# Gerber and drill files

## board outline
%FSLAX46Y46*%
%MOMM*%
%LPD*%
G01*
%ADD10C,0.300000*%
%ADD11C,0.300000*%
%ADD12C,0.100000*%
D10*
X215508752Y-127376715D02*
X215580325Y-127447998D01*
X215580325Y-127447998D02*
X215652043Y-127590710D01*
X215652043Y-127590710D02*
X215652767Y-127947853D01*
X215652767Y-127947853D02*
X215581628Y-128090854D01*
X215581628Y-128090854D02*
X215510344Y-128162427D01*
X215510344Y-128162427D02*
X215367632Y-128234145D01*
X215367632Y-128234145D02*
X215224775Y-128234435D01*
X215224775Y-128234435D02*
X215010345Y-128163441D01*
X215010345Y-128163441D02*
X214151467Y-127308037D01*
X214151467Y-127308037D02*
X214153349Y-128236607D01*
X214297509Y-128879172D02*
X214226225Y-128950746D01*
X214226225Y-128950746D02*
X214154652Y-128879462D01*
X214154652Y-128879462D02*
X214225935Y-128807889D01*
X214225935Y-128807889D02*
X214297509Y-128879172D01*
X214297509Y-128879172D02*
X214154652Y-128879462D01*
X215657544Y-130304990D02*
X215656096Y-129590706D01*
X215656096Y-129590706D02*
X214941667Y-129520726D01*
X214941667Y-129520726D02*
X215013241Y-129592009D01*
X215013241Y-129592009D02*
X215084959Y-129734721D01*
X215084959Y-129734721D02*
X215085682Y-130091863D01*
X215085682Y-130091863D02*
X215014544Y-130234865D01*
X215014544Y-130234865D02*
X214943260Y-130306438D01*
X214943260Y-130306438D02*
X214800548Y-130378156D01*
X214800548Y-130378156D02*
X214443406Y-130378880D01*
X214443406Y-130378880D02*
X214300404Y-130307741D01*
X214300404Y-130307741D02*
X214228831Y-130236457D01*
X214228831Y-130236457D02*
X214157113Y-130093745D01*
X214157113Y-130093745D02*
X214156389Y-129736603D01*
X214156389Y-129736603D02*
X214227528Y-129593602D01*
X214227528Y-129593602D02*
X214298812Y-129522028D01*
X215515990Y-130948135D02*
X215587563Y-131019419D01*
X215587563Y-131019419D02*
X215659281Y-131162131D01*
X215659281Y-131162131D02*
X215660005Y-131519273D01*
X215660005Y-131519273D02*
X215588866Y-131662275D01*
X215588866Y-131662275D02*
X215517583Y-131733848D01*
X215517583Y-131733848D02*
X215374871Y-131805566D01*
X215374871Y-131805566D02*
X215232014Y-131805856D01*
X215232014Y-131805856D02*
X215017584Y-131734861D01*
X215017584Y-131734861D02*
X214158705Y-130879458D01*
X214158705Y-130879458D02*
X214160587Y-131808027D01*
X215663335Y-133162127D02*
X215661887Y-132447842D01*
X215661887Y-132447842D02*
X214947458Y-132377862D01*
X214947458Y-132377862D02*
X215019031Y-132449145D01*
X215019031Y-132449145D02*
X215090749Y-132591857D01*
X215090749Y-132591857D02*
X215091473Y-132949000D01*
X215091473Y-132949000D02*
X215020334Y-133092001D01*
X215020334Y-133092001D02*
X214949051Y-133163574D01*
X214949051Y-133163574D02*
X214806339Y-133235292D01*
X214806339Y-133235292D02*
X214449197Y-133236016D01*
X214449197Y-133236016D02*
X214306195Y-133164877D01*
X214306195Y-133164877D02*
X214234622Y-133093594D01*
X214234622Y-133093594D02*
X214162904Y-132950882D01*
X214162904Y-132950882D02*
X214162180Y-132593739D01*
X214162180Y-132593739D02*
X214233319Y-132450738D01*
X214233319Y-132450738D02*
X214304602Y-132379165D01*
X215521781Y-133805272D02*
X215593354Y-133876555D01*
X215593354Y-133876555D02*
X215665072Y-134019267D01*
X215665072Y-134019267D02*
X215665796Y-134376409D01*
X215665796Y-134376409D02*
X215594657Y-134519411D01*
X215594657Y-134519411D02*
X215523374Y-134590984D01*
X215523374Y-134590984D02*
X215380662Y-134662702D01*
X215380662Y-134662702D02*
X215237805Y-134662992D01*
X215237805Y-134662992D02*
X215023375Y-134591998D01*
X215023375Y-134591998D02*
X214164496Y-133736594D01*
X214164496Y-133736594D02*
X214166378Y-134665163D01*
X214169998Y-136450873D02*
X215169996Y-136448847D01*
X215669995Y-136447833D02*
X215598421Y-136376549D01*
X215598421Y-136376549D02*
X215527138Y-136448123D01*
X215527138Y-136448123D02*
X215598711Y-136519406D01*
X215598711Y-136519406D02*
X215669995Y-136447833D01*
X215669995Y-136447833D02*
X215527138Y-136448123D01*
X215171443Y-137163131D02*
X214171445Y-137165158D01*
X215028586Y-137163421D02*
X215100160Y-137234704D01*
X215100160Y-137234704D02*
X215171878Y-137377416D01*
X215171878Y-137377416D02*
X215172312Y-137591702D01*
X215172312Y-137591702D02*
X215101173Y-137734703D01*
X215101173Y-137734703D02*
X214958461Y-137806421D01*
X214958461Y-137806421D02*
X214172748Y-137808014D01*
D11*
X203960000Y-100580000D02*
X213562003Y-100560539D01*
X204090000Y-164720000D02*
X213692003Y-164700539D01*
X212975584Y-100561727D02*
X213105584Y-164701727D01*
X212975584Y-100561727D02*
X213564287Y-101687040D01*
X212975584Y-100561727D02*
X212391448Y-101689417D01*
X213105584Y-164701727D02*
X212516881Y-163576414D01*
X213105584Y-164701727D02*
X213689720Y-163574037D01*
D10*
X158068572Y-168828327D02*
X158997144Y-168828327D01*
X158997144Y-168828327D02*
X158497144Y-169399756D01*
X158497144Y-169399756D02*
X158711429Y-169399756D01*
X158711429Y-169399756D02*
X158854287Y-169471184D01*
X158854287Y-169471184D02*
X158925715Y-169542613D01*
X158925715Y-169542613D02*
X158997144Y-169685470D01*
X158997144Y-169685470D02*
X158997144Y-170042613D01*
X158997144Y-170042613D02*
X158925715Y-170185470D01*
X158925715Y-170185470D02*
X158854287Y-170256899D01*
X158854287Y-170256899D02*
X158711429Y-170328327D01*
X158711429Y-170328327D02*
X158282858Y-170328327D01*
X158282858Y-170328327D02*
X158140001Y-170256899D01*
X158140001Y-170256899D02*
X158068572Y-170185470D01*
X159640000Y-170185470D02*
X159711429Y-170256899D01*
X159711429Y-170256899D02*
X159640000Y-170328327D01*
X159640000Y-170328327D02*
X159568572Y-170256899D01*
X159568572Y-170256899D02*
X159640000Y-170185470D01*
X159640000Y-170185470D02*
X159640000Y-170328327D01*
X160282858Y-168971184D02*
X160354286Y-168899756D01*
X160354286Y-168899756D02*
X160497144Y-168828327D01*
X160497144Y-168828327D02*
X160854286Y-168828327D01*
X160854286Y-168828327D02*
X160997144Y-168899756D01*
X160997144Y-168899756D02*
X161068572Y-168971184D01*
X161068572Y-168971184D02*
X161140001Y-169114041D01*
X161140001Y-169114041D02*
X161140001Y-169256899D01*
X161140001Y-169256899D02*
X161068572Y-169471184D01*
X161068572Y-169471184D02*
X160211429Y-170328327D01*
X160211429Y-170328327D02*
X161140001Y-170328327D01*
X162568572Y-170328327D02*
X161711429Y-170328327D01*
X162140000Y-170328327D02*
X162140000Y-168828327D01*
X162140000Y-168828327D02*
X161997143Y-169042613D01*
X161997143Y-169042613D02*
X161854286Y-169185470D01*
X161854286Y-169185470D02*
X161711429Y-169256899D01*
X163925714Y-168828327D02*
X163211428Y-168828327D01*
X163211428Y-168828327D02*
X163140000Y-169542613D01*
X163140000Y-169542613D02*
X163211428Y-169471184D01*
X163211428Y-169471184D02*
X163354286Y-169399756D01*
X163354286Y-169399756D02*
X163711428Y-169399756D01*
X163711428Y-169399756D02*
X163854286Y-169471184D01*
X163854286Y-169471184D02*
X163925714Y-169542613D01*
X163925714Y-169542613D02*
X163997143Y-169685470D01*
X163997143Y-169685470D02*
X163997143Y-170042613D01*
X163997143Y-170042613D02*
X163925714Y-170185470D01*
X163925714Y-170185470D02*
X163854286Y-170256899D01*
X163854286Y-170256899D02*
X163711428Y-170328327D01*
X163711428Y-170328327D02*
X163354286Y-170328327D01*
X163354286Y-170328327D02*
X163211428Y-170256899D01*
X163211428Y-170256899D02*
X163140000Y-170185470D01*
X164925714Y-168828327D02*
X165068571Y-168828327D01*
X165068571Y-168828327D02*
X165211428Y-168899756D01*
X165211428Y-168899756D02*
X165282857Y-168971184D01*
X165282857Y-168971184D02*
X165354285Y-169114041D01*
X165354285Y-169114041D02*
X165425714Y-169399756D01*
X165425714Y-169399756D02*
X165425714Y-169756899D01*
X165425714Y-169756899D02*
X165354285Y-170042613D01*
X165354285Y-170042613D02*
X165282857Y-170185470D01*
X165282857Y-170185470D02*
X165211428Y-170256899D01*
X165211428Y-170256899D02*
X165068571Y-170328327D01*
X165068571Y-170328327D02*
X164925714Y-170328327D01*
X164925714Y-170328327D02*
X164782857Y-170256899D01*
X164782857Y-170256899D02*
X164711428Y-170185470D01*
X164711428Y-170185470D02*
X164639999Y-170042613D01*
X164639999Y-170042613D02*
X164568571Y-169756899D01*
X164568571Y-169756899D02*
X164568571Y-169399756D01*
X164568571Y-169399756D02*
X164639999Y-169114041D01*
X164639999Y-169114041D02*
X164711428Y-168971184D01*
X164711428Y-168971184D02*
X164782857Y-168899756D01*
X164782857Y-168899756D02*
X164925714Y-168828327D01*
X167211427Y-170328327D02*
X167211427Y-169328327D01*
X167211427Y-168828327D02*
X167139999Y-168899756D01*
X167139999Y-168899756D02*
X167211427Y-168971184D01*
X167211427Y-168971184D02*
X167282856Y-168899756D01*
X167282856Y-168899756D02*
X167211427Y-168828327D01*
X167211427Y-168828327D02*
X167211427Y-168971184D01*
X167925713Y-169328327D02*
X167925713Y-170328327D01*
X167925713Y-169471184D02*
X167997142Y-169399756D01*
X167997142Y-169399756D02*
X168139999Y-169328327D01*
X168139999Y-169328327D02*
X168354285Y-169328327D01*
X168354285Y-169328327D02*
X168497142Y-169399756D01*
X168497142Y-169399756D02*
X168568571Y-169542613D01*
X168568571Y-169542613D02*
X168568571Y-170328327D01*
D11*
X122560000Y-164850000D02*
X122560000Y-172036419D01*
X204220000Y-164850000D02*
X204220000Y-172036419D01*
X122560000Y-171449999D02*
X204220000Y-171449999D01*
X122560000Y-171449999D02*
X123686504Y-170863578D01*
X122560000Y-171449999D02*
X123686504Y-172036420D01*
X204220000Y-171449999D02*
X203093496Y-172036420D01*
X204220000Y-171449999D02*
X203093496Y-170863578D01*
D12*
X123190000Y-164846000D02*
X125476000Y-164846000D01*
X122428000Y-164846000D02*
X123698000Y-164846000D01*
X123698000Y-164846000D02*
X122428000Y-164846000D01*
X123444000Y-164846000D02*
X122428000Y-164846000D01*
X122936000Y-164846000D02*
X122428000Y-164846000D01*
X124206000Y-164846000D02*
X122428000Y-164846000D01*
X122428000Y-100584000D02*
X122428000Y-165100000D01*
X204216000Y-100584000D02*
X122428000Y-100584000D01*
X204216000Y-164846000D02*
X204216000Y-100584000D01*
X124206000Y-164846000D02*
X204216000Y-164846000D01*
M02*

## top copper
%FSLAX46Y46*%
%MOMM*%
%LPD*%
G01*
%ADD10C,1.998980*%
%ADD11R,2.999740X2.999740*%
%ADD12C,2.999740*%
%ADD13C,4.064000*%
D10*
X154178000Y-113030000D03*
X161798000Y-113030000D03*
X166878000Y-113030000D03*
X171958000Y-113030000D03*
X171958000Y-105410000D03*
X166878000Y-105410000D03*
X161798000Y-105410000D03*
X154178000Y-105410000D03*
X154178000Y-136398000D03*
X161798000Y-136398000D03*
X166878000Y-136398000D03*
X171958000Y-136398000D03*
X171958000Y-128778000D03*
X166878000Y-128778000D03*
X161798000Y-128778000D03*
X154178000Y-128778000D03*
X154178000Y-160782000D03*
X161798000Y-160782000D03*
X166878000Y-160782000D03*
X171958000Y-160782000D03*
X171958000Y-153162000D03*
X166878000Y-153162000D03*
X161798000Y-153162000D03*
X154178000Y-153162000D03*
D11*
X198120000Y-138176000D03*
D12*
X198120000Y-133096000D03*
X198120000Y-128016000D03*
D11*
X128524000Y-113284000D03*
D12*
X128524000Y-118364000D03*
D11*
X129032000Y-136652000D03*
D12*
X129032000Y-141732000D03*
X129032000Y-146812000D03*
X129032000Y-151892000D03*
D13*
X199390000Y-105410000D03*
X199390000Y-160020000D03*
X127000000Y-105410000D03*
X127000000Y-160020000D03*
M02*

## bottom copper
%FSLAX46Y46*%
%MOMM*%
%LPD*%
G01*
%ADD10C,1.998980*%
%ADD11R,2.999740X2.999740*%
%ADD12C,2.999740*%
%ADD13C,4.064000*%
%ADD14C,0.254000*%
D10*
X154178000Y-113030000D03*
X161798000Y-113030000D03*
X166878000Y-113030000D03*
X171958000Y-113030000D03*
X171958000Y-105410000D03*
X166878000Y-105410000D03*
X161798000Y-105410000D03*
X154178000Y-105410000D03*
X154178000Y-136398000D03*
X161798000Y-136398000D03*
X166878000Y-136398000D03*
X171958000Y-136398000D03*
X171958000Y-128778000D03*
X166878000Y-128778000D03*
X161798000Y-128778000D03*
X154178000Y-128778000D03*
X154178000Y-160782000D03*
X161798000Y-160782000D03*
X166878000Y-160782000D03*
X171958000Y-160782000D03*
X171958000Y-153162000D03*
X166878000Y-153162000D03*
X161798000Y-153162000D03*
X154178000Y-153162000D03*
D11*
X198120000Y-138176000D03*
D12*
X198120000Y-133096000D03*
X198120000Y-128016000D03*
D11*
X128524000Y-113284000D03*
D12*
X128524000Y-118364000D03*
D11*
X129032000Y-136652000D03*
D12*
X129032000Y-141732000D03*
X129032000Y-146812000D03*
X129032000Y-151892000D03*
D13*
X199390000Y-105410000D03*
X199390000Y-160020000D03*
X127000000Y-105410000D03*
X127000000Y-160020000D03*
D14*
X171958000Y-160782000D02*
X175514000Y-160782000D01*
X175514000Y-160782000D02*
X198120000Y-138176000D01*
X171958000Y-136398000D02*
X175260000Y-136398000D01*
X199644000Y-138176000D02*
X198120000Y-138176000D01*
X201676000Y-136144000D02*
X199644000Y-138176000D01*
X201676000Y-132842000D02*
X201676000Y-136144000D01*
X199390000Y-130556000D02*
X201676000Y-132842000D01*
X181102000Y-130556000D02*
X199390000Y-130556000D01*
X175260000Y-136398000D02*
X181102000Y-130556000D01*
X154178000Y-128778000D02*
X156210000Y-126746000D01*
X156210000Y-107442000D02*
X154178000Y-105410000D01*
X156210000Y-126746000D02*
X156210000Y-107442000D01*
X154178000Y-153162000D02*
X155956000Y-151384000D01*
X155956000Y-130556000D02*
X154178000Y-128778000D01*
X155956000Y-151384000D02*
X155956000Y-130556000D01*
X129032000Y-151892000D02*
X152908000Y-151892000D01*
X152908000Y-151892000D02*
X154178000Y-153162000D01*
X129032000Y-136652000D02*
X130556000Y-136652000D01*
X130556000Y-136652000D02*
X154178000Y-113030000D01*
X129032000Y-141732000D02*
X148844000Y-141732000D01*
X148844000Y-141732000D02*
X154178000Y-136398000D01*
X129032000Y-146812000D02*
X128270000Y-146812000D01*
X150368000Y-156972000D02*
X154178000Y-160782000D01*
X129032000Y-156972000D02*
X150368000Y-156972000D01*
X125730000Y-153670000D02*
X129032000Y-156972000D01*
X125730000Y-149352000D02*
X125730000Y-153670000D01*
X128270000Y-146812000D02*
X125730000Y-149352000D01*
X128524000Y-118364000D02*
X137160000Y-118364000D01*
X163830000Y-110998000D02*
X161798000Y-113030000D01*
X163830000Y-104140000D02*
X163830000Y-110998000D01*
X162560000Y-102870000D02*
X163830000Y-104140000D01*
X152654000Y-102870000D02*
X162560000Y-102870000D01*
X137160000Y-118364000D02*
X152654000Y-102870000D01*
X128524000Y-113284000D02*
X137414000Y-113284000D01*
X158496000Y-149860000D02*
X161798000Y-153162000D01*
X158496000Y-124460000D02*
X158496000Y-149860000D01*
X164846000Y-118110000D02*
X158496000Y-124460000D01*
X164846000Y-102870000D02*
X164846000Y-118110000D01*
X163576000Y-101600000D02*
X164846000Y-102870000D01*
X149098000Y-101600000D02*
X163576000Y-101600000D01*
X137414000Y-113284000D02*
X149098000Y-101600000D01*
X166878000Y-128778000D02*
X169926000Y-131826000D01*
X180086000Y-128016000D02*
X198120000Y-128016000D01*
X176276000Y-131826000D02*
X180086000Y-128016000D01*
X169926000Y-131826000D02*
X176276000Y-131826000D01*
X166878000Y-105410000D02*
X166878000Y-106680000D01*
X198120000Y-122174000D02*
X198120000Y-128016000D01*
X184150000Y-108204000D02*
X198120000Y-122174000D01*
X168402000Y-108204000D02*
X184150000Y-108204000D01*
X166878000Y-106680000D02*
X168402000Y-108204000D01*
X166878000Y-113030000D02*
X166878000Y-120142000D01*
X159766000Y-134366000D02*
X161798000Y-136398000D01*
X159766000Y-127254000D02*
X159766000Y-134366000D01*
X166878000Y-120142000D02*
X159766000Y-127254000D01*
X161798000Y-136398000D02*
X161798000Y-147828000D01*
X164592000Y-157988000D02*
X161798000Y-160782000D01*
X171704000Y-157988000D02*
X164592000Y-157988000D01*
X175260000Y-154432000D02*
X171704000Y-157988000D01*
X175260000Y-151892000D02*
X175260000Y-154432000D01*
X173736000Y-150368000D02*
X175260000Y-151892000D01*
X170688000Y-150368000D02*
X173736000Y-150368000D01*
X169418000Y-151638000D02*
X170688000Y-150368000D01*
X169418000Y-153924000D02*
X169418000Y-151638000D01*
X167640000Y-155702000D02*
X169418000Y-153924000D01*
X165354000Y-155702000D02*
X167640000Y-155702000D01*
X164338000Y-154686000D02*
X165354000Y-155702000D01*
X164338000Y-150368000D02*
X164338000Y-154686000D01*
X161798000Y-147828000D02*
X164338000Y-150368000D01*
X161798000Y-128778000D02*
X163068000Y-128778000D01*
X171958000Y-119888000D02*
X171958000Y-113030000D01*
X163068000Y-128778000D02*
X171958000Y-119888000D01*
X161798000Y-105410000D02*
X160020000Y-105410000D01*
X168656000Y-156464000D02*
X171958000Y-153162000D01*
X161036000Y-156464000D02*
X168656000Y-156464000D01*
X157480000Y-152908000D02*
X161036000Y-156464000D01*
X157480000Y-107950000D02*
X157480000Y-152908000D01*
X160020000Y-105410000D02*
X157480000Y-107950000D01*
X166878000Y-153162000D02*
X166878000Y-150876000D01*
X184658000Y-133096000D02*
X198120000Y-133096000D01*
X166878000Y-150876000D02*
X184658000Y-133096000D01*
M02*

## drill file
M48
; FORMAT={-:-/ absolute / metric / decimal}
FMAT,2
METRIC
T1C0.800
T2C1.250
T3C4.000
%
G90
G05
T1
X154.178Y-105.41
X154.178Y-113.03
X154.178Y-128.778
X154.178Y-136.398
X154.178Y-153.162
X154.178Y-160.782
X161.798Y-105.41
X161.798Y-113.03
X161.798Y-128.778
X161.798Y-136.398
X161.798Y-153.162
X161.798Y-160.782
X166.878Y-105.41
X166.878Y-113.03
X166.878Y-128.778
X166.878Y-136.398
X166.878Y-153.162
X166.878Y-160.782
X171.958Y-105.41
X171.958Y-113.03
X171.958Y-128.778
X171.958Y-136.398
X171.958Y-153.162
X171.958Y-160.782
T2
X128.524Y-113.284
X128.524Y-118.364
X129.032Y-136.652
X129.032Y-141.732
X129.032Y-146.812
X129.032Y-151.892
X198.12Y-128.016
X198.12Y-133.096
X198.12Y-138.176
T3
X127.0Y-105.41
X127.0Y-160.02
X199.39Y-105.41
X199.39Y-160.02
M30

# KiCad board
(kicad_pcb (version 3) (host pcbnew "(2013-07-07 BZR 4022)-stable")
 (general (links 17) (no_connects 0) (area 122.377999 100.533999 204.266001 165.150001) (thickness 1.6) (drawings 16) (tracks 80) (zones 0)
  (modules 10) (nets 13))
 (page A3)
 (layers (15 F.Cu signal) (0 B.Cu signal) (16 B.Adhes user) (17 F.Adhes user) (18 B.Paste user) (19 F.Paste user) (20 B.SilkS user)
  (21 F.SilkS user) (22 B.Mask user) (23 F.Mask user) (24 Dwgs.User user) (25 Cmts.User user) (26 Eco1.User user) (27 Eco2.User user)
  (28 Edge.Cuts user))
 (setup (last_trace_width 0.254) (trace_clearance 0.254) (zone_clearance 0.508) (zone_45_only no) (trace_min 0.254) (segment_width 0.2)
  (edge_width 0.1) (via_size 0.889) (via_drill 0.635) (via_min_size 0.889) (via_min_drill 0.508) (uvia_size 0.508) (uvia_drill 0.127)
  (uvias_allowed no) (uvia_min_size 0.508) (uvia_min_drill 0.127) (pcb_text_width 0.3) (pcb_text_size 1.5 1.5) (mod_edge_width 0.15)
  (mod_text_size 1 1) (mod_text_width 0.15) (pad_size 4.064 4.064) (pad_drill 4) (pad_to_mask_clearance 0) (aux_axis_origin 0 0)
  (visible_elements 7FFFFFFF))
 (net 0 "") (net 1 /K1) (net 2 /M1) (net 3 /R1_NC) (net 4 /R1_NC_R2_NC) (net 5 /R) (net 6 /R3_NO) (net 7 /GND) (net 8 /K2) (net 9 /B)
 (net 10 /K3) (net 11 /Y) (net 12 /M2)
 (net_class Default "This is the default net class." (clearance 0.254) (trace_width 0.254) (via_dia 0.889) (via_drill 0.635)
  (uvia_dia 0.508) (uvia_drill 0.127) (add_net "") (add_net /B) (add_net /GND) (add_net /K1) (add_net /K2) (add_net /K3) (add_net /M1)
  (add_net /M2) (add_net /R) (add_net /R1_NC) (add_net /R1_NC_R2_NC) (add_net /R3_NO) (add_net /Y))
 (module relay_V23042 (layer F.Cu) (at 163.068 109.22)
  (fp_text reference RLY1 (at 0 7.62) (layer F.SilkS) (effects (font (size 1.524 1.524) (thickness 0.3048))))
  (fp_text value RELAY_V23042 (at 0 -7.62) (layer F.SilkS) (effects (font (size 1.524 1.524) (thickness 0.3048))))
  (pad 1 thru_hole circle (at -8.89 3.81) (size 1.99898 1.99898) (drill 0.8001) (layers *.Cu *.Mask F.SilkS) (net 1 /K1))
  (pad 4 thru_hole circle (at -1.27 3.81) (size 1.99898 1.99898) (drill 0.8001) (layers *.Cu *.Mask F.SilkS) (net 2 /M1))
  (pad 6 thru_hole circle (at 3.81 3.81) (size 1.99898 1.99898) (drill 0.8001) (layers *.Cu *.Mask F.SilkS) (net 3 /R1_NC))
  (pad 8 thru_hole circle (at 8.89 3.81) (size 1.99898 1.99898) (drill 0.8001) (layers *.Cu *.Mask F.SilkS) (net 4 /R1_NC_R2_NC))
  (pad 9 thru_hole circle (at 8.89 -3.81) (size 1.99898 1.99898) (drill 0.8001) (layers *.Cu *.Mask F.SilkS))
  (pad 11 thru_hole circle (at 3.81 -3.81) (size 1.99898 1.99898) (drill 0.8001) (layers *.Cu *.Mask F.SilkS) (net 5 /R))
  (pad 13 thru_hole circle (at -1.27 -3.81) (size 1.99898 1.99898) (drill 0.8001) (layers *.Cu *.Mask F.SilkS) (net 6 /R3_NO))
  (pad 16 thru_hole circle (at -8.89 -3.81) (size 1.99898 1.99898) (drill 0.8001) (layers *.Cu *.Mask F.SilkS) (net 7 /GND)))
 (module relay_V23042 (layer F.Cu) (at 163.068 132.588)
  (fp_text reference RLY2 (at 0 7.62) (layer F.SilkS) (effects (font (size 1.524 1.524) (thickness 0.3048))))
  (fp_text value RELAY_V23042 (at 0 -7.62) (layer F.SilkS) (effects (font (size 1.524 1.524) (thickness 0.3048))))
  (pad 1 thru_hole circle (at -8.89 3.81) (size 1.99898 1.99898) (drill 0.8001) (layers *.Cu *.Mask F.SilkS) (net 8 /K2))
  (pad 4 thru_hole circle (at -1.27 3.81) (size 1.99898 1.99898) (drill 0.8001) (layers *.Cu *.Mask F.SilkS) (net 3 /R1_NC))
  (pad 6 thru_hole circle (at 3.81 3.81) (size 1.99898 1.99898) (drill 0.8001) (layers *.Cu *.Mask F.SilkS))
  (pad 8 thru_hole circle (at 8.89 3.81) (size 1.99898 1.99898) (drill 0.8001) (layers *.Cu *.Mask F.SilkS) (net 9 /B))
  (pad 9 thru_hole circle (at 8.89 -3.81) (size 1.99898 1.99898) (drill 0.8001) (layers *.Cu *.Mask F.SilkS))
  (pad 11 thru_hole circle (at 3.81 -3.81) (size 1.99898 1.99898) (drill 0.8001) (layers *.Cu *.Mask F.SilkS) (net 5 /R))
  (pad 13 thru_hole circle (at -1.27 -3.81) (size 1.99898 1.99898) (drill 0.8001) (layers *.Cu *.Mask F.SilkS) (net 4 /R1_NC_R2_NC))
  (pad 16 thru_hole circle (at -8.89 -3.81) (size 1.99898 1.99898) (drill 0.8001) (layers *.Cu *.Mask F.SilkS) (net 7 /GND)))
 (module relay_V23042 (layer F.Cu) (at 163.068 156.972)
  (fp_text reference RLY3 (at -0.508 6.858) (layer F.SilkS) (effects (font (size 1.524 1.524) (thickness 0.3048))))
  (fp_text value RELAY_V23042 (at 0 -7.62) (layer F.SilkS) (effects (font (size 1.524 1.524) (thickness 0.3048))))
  (pad 1 thru_hole circle (at -8.89 3.81) (size 1.99898 1.99898) (drill 0.8001) (layers *.Cu *.Mask F.SilkS) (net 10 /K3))
  (pad 4 thru_hole circle (at -1.27 3.81) (size 1.99898 1.99898) (drill 0.8001) (layers *.Cu *.Mask F.SilkS) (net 3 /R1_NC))
  (pad 6 thru_hole circle (at 3.81 3.81) (size 1.99898 1.99898) (drill 0.8001) (layers *.Cu *.Mask F.SilkS))
  (pad 8 thru_hole circle (at 8.89 3.81) (size 1.99898 1.99898) (drill 0.8001) (layers *.Cu *.Mask F.SilkS) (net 9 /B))
  (pad 9 thru_hole circle (at 8.89 -3.81) (size 1.99898 1.99898) (drill 0.8001) (layers *.Cu *.Mask F.SilkS) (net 6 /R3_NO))
  (pad 11 thru_hole circle (at 3.81 -3.81) (size 1.99898 1.99898) (drill 0.8001) (layers *.Cu *.Mask F.SilkS) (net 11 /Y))
  (pad 13 thru_hole circle (at -1.27 -3.81) (size 1.99898 1.99898) (drill 0.8001) (layers *.Cu *.Mask F.SilkS) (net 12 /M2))
  (pad 16 thru_hole circle (at -8.89 -3.81) (size 1.99898 1.99898) (drill 0.8001) (layers *.Cu *.Mask F.SilkS) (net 7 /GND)))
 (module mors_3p (layer F.Cu) (at 198.12 133.096 90)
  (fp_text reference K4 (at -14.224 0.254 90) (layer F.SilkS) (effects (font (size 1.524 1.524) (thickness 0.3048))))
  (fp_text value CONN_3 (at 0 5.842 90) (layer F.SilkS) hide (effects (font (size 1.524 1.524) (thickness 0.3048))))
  (pad 1 thru_hole rect (at -5.08 0 90) (size 2.99974 2.99974) (drill 1.24968) (layers *.Cu *.Mask F.SilkS) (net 9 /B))
  (pad 2 thru_hole circle (at 0 0 90) (size 2.99974 2.99974) (drill 1.24968) (layers *.Cu *.Mask F.SilkS) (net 11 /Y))
  (pad 3 thru_hole circle (at 5.08 0 90) (size 2.99974 2.99974) (drill 1.24968) (layers *.Cu *.Mask F.SilkS) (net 5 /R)))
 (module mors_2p (layer F.Cu) (at 128.524 115.824 270)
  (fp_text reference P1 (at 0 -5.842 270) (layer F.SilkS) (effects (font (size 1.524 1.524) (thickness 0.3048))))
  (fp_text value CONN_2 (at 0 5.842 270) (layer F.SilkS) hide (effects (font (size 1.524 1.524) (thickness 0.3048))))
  (pad 1 thru_hole rect (at -2.54 0 270) (size 2.99974 2.99974) (drill 1.24968) (layers *.Cu *.Mask F.SilkS) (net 12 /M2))
  (pad 2 thru_hole circle (at 2.54 0 270) (size 2.99974 2.99974) (drill 1.24968) (layers *.Cu *.Mask F.SilkS) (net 2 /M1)))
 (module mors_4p (layer F.Cu) (at 129.032 144.272 270)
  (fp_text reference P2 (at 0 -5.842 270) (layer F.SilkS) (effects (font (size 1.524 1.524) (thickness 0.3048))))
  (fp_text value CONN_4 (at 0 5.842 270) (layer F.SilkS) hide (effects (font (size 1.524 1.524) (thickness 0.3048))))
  (pad 1 thru_hole rect (at -7.62 0 270) (size 2.99974 2.99974) (drill 1.24968) (layers *.Cu *.Mask F.SilkS) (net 1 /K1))
  (pad 2 thru_hole circle (at -2.54 0 270) (size 2.99974 2.99974) (drill 1.24968) (layers *.Cu *.Mask F.SilkS) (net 8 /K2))
  (pad 3 thru_hole circle (at 2.54 0 270) (size 2.99974 2.99974) (drill 1.24968) (layers *.Cu *.Mask F.SilkS) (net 10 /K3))
  (pad 4 thru_hole circle (at 7.62 0 270) (size 2.99974 2.99974) (drill 1.24968) (layers *.Cu *.Mask F.SilkS) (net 7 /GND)))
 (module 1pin (layer F.Cu) (at 199.39 105.41)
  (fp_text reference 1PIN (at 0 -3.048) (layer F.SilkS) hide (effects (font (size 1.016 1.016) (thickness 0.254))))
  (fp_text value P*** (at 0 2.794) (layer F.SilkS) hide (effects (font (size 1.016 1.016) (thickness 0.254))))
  (pad 1 thru_hole circle (at 0 0) (size 4.064 4.064) (drill 4) (layers *.Cu *.Mask F.SilkS)))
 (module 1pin (layer F.Cu) (at 199.39 160.02)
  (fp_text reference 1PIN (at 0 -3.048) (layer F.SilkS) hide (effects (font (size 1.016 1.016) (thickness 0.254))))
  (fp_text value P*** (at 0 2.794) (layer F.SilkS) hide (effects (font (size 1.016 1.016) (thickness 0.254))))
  (pad 1 thru_hole circle (at 0 0) (size 4.064 4.064) (drill 4) (layers *.Cu *.Mask F.SilkS)))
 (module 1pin (layer F.Cu) (at 127 105.41)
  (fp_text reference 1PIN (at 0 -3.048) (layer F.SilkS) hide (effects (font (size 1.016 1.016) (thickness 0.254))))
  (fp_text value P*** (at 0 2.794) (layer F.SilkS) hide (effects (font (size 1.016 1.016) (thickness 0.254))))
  (pad 1 thru_hole circle (at 0 0) (size 4.064 4.064) (drill 4) (layers *.Cu *.Mask F.SilkS)))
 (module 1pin (layer F.Cu) (at 127 160.02)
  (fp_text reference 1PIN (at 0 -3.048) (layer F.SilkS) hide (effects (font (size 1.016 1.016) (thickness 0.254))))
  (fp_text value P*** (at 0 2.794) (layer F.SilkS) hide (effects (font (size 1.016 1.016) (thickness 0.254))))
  (pad 1 thru_hole circle (at 0 0) (size 4.064 4.064) (drill 4) (layers *.Cu *.Mask F.SilkS)))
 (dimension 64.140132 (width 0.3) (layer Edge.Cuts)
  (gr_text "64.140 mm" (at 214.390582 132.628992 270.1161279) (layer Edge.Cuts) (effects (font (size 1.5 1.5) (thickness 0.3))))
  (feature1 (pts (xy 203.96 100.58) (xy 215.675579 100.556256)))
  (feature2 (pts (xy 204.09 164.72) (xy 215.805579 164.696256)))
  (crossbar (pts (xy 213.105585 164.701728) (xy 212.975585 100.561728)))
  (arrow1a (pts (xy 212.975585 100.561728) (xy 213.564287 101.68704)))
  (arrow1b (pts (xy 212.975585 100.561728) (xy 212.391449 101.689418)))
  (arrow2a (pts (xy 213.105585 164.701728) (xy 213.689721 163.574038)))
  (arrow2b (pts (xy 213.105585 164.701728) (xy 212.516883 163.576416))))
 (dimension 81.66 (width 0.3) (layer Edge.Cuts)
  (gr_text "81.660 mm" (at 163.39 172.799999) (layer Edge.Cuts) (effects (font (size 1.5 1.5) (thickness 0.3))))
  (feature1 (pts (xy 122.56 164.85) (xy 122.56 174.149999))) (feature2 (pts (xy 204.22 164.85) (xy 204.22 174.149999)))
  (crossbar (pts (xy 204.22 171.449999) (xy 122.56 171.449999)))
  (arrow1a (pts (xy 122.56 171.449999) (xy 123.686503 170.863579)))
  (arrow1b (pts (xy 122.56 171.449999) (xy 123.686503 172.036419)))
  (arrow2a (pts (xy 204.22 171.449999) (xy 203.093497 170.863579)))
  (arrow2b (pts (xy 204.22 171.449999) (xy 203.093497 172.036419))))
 (gr_line (start 123.19 164.846) (end 125.476 164.846) (angle 90) (layer Edge.Cuts) (width 0.1))
 (gr_line (start 122.428 164.846) (end 123.698 164.846) (angle 90) (layer Edge.Cuts) (width 0.1))
 (gr_line (start 123.698 164.846) (end 122.428 164.846) (angle 90) (layer Edge.Cuts) (width 0.1))
 (gr_line (start 123.444 164.846) (end 122.428 164.846) (angle 90) (layer Edge.Cuts) (width 0.1))
 (gr_line (start 122.936 164.846) (end 122.428 164.846) (angle 90) (layer Edge.Cuts) (width 0.1))
 (gr_line (start 124.206 164.846) (end 122.428 164.846) (angle 90) (layer Edge.Cuts) (width 0.1))
 (gr_line (start 122.428 100.584) (end 122.428 165.1) (angle 90) (layer Edge.Cuts) (width 0.1))
 (gr_line (start 204.216 100.584) (end 122.428 100.584) (angle 90) (layer Edge.Cuts) (width 0.1))
 (gr_line (start 204.216 164.846) (end 204.216 100.584) (angle 90) (layer Edge.Cuts) (width 0.1))
 (gr_line (start 124.206 164.846) (end 204.216 164.846) (angle 90) (layer Edge.Cuts) (width 0.1))
 (segment (start 171.958 160.782) (end 175.514 160.782) (width 0.254) (layer B.Cu) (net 9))
 (segment (start 175.514 160.782) (end 198.12 138.176) (width 0.254) (layer B.Cu) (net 9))
 (segment (start 171.958 136.398) (end 175.26 136.398) (width 0.254) (layer B.Cu) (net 9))
 (segment (start 199.644 138.176) (end 198.12 138.176) (width 0.254) (layer B.Cu) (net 9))
 (segment (start 201.676 136.144) (end 199.644 138.176) (width 0.254) (layer B.Cu) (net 9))
 (segment (start 201.676 132.842) (end 201.676 136.144) (width 0.254) (layer B.Cu) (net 9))
 (segment (start 199.39 130.556) (end 201.676 132.842) (width 0.254) (layer B.Cu) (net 9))
 (segment (start 181.102 130.556) (end 199.39 130.556) (width 0.254) (layer B.Cu) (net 9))
 (segment (start 175.26 136.398) (end 181.102 130.556) (width 0.254) (layer B.Cu) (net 9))
 (segment (start 154.178 128.778) (end 156.21 126.746) (width 0.254) (layer B.Cu) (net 7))
 (segment (start 156.21 107.442) (end 154.178 105.41) (width 0.254) (layer B.Cu) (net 7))
 (segment (start 156.21 126.746) (end 156.21 107.442) (width 0.254) (layer B.Cu) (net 7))
 (segment (start 154.178 153.162) (end 155.956 151.384) (width 0.254) (layer B.Cu) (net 7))
 (segment (start 155.956 130.556) (end 154.178 128.778) (width 0.254) (layer B.Cu) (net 7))
 (segment (start 155.956 151.384) (end 155.956 130.556) (width 0.254) (layer B.Cu) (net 7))
 (segment (start 129.032 151.892) (end 152.908 151.892) (width 0.254) (layer B.Cu) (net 7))
 (segment (start 152.908 151.892) (end 154.178 153.162) (width 0.254) (layer B.Cu) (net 7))
 (segment (start 129.032 136.652) (end 130.556 136.652) (width 0.254) (layer B.Cu) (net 1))
 (segment (start 130.556 136.652) (end 154.178 113.03) (width 0.254) (layer B.Cu) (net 1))
 (segment (start 129.032 141.732) (end 148.844 141.732) (width 0.254) (layer B.Cu) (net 8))
 (segment (start 148.844 141.732) (end 154.178 136.398) (width 0.254) (layer B.Cu) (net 8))
 (segment (start 129.032 146.812) (end 128.27 146.812) (width 0.254) (layer B.Cu) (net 10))
 (segment (start 150.368 156.972) (end 154.178 160.782) (width 0.254) (layer B.Cu) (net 10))
 (segment (start 129.032 156.972) (end 150.368 156.972) (width 0.254) (layer B.Cu) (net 10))
 (segment (start 125.73 153.67) (end 129.032 156.972) (width 0.254) (layer B.Cu) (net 10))
 (segment (start 125.73 149.352) (end 125.73 153.67) (width 0.254) (layer B.Cu) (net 10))
 (segment (start 128.27 146.812) (end 125.73 149.352) (width 0.254) (layer B.Cu) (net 10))
 (segment (start 128.524 118.364) (end 137.16 118.364) (width 0.254) (layer B.Cu) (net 2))
 (segment (start 163.83 110.998) (end 161.798 113.03) (width 0.254) (layer B.Cu) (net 2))
 (segment (start 163.83 104.14) (end 163.83 110.998) (width 0.254) (layer B.Cu) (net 2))
 (segment (start 162.56 102.87) (end 163.83 104.14) (width 0.254) (layer B.Cu) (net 2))
 (segment (start 152.654 102.87) (end 162.56 102.87) (width 0.254) (layer B.Cu) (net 2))
 (segment (start 137.16 118.364) (end 152.654 102.87) (width 0.254) (layer B.Cu) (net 2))
 (segment (start 128.524 113.284) (end 137.414 113.284) (width 0.254) (layer B.Cu) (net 12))
 (segment (start 158.496 149.86) (end 161.798 153.162) (width 0.254) (layer B.Cu) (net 12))
 (segment (start 158.496 124.46) (end 158.496 149.86) (width 0.254) (layer B.Cu) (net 12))
 (segment (start 164.846 118.11) (end 158.496 124.46) (width 0.254) (layer B.Cu) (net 12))
 (segment (start 164.846 102.87) (end 164.846 118.11) (width 0.254) (layer B.Cu) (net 12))
 (segment (start 163.576 101.6) (end 164.846 102.87) (width 0.254) (layer B.Cu) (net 12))
 (segment (start 149.098 101.6) (end 163.576 101.6) (width 0.254) (layer B.Cu) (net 12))
 (segment (start 137.414 113.284) (end 149.098 101.6) (width 0.254) (layer B.Cu) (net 12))
 (segment (start 166.878 128.778) (end 169.926 131.826) (width 0.254) (layer B.Cu) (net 5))
 (segment (start 180.086 128.016) (end 198.12 128.016) (width 0.254) (layer B.Cu) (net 5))
 (segment (start 176.276 131.826) (end 180.086 128.016) (width 0.254) (layer B.Cu) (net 5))
 (segment (start 169.926 131.826) (end 176.276 131.826) (width 0.254) (layer B.Cu) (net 5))
 (segment (start 166.878 105.41) (end 166.878 106.68) (width 0.254) (layer B.Cu) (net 5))
 (segment (start 198.12 122.174) (end 198.12 128.016) (width 0.254) (layer B.Cu) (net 5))
 (segment (start 184.15 108.204) (end 198.12 122.174) (width 0.254) (layer B.Cu) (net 5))
 (segment (start 168.402 108.204) (end 184.15 108.204) (width 0.254) (layer B.Cu) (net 5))
 (segment (start 166.878 106.68) (end 168.402 108.204) (width 0.254) (layer B.Cu) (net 5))
 (segment (start 166.878 113.03) (end 166.878 120.142) (width 0.254) (layer B.Cu) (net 3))
 (segment (start 159.766 134.366) (end 161.798 136.398) (width 0.254) (layer B.Cu) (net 3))
 (segment (start 159.766 127.254) (end 159.766 134.366) (width 0.254) (layer B.Cu) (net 3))
 (segment (start 166.878 120.142) (end 159.766 127.254) (width 0.254) (layer B.Cu) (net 3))
 (segment (start 161.798 136.398) (end 161.798 147.828) (width 0.254) (layer B.Cu) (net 3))
 (segment (start 164.592 157.988) (end 161.798 160.782) (width 0.254) (layer B.Cu) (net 3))
 (segment (start 171.704 157.988) (end 164.592 157.988) (width 0.254) (layer B.Cu) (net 3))
 (segment (start 175.26 154.432) (end 171.704 157.988) (width 0.254) (layer B.Cu) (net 3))
 (segment (start 175.26 151.892) (end 175.26 154.432) (width 0.254) (layer B.Cu) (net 3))
 (segment (start 173.736 150.368) (end 175.26 151.892) (width 0.254) (layer B.Cu) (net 3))
 (segment (start 170.688 150.368) (end 173.736 150.368) (width 0.254) (layer B.Cu) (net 3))
 (segment (start 169.418 151.638) (end 170.688 150.368) (width 0.254) (layer B.Cu) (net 3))
 (segment (start 169.418 153.924) (end 169.418 151.638) (width 0.254) (layer B.Cu) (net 3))
 (segment (start 167.64 155.702) (end 169.418 153.924) (width 0.254) (layer B.Cu) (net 3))
 (segment (start 165.354 155.702) (end 167.64 155.702) (width 0.254) (layer B.Cu) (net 3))
 (segment (start 164.338 154.686) (end 165.354 155.702) (width 0.254) (layer B.Cu) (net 3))
 (segment (start 164.338 150.368) (end 164.338 154.686) (width 0.254) (layer B.Cu) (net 3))
 (segment (start 161.798 147.828) (end 164.338 150.368) (width 0.254) (layer B.Cu) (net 3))
 (segment (start 161.798 128.778) (end 163.068 128.778) (width 0.254) (layer B.Cu) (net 4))
 (segment (start 171.958 119.888) (end 171.958 113.03) (width 0.254) (layer B.Cu) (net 4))
 (segment (start 163.068 128.778) (end 171.958 119.888) (width 0.254) (layer B.Cu) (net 4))
 (segment (start 161.798 105.41) (end 160.02 105.41) (width 0.254) (layer B.Cu) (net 6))
 (segment (start 168.656 156.464) (end 171.958 153.162) (width 0.254) (layer B.Cu) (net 6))
 (segment (start 161.036 156.464) (end 168.656 156.464) (width 0.254) (layer B.Cu) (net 6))
 (segment (start 157.48 152.908) (end 161.036 156.464) (width 0.254) (layer B.Cu) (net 6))
 (segment (start 157.48 107.95) (end 157.48 152.908) (width 0.254) (layer B.Cu) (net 6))
 (segment (start 160.02 105.41) (end 157.48 107.95) (width 0.254) (layer B.Cu) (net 6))
 (segment (start 166.878 153.162) (end 166.878 150.876) (width 0.254) (layer B.Cu) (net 11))
 (segment (start 184.658 133.096) (end 198.12 133.096) (width 0.254) (layer B.Cu) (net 11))
 (segment (start 166.878 150.876) (end 184.658 133.096) (width 0.254) (layer B.Cu) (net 11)))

